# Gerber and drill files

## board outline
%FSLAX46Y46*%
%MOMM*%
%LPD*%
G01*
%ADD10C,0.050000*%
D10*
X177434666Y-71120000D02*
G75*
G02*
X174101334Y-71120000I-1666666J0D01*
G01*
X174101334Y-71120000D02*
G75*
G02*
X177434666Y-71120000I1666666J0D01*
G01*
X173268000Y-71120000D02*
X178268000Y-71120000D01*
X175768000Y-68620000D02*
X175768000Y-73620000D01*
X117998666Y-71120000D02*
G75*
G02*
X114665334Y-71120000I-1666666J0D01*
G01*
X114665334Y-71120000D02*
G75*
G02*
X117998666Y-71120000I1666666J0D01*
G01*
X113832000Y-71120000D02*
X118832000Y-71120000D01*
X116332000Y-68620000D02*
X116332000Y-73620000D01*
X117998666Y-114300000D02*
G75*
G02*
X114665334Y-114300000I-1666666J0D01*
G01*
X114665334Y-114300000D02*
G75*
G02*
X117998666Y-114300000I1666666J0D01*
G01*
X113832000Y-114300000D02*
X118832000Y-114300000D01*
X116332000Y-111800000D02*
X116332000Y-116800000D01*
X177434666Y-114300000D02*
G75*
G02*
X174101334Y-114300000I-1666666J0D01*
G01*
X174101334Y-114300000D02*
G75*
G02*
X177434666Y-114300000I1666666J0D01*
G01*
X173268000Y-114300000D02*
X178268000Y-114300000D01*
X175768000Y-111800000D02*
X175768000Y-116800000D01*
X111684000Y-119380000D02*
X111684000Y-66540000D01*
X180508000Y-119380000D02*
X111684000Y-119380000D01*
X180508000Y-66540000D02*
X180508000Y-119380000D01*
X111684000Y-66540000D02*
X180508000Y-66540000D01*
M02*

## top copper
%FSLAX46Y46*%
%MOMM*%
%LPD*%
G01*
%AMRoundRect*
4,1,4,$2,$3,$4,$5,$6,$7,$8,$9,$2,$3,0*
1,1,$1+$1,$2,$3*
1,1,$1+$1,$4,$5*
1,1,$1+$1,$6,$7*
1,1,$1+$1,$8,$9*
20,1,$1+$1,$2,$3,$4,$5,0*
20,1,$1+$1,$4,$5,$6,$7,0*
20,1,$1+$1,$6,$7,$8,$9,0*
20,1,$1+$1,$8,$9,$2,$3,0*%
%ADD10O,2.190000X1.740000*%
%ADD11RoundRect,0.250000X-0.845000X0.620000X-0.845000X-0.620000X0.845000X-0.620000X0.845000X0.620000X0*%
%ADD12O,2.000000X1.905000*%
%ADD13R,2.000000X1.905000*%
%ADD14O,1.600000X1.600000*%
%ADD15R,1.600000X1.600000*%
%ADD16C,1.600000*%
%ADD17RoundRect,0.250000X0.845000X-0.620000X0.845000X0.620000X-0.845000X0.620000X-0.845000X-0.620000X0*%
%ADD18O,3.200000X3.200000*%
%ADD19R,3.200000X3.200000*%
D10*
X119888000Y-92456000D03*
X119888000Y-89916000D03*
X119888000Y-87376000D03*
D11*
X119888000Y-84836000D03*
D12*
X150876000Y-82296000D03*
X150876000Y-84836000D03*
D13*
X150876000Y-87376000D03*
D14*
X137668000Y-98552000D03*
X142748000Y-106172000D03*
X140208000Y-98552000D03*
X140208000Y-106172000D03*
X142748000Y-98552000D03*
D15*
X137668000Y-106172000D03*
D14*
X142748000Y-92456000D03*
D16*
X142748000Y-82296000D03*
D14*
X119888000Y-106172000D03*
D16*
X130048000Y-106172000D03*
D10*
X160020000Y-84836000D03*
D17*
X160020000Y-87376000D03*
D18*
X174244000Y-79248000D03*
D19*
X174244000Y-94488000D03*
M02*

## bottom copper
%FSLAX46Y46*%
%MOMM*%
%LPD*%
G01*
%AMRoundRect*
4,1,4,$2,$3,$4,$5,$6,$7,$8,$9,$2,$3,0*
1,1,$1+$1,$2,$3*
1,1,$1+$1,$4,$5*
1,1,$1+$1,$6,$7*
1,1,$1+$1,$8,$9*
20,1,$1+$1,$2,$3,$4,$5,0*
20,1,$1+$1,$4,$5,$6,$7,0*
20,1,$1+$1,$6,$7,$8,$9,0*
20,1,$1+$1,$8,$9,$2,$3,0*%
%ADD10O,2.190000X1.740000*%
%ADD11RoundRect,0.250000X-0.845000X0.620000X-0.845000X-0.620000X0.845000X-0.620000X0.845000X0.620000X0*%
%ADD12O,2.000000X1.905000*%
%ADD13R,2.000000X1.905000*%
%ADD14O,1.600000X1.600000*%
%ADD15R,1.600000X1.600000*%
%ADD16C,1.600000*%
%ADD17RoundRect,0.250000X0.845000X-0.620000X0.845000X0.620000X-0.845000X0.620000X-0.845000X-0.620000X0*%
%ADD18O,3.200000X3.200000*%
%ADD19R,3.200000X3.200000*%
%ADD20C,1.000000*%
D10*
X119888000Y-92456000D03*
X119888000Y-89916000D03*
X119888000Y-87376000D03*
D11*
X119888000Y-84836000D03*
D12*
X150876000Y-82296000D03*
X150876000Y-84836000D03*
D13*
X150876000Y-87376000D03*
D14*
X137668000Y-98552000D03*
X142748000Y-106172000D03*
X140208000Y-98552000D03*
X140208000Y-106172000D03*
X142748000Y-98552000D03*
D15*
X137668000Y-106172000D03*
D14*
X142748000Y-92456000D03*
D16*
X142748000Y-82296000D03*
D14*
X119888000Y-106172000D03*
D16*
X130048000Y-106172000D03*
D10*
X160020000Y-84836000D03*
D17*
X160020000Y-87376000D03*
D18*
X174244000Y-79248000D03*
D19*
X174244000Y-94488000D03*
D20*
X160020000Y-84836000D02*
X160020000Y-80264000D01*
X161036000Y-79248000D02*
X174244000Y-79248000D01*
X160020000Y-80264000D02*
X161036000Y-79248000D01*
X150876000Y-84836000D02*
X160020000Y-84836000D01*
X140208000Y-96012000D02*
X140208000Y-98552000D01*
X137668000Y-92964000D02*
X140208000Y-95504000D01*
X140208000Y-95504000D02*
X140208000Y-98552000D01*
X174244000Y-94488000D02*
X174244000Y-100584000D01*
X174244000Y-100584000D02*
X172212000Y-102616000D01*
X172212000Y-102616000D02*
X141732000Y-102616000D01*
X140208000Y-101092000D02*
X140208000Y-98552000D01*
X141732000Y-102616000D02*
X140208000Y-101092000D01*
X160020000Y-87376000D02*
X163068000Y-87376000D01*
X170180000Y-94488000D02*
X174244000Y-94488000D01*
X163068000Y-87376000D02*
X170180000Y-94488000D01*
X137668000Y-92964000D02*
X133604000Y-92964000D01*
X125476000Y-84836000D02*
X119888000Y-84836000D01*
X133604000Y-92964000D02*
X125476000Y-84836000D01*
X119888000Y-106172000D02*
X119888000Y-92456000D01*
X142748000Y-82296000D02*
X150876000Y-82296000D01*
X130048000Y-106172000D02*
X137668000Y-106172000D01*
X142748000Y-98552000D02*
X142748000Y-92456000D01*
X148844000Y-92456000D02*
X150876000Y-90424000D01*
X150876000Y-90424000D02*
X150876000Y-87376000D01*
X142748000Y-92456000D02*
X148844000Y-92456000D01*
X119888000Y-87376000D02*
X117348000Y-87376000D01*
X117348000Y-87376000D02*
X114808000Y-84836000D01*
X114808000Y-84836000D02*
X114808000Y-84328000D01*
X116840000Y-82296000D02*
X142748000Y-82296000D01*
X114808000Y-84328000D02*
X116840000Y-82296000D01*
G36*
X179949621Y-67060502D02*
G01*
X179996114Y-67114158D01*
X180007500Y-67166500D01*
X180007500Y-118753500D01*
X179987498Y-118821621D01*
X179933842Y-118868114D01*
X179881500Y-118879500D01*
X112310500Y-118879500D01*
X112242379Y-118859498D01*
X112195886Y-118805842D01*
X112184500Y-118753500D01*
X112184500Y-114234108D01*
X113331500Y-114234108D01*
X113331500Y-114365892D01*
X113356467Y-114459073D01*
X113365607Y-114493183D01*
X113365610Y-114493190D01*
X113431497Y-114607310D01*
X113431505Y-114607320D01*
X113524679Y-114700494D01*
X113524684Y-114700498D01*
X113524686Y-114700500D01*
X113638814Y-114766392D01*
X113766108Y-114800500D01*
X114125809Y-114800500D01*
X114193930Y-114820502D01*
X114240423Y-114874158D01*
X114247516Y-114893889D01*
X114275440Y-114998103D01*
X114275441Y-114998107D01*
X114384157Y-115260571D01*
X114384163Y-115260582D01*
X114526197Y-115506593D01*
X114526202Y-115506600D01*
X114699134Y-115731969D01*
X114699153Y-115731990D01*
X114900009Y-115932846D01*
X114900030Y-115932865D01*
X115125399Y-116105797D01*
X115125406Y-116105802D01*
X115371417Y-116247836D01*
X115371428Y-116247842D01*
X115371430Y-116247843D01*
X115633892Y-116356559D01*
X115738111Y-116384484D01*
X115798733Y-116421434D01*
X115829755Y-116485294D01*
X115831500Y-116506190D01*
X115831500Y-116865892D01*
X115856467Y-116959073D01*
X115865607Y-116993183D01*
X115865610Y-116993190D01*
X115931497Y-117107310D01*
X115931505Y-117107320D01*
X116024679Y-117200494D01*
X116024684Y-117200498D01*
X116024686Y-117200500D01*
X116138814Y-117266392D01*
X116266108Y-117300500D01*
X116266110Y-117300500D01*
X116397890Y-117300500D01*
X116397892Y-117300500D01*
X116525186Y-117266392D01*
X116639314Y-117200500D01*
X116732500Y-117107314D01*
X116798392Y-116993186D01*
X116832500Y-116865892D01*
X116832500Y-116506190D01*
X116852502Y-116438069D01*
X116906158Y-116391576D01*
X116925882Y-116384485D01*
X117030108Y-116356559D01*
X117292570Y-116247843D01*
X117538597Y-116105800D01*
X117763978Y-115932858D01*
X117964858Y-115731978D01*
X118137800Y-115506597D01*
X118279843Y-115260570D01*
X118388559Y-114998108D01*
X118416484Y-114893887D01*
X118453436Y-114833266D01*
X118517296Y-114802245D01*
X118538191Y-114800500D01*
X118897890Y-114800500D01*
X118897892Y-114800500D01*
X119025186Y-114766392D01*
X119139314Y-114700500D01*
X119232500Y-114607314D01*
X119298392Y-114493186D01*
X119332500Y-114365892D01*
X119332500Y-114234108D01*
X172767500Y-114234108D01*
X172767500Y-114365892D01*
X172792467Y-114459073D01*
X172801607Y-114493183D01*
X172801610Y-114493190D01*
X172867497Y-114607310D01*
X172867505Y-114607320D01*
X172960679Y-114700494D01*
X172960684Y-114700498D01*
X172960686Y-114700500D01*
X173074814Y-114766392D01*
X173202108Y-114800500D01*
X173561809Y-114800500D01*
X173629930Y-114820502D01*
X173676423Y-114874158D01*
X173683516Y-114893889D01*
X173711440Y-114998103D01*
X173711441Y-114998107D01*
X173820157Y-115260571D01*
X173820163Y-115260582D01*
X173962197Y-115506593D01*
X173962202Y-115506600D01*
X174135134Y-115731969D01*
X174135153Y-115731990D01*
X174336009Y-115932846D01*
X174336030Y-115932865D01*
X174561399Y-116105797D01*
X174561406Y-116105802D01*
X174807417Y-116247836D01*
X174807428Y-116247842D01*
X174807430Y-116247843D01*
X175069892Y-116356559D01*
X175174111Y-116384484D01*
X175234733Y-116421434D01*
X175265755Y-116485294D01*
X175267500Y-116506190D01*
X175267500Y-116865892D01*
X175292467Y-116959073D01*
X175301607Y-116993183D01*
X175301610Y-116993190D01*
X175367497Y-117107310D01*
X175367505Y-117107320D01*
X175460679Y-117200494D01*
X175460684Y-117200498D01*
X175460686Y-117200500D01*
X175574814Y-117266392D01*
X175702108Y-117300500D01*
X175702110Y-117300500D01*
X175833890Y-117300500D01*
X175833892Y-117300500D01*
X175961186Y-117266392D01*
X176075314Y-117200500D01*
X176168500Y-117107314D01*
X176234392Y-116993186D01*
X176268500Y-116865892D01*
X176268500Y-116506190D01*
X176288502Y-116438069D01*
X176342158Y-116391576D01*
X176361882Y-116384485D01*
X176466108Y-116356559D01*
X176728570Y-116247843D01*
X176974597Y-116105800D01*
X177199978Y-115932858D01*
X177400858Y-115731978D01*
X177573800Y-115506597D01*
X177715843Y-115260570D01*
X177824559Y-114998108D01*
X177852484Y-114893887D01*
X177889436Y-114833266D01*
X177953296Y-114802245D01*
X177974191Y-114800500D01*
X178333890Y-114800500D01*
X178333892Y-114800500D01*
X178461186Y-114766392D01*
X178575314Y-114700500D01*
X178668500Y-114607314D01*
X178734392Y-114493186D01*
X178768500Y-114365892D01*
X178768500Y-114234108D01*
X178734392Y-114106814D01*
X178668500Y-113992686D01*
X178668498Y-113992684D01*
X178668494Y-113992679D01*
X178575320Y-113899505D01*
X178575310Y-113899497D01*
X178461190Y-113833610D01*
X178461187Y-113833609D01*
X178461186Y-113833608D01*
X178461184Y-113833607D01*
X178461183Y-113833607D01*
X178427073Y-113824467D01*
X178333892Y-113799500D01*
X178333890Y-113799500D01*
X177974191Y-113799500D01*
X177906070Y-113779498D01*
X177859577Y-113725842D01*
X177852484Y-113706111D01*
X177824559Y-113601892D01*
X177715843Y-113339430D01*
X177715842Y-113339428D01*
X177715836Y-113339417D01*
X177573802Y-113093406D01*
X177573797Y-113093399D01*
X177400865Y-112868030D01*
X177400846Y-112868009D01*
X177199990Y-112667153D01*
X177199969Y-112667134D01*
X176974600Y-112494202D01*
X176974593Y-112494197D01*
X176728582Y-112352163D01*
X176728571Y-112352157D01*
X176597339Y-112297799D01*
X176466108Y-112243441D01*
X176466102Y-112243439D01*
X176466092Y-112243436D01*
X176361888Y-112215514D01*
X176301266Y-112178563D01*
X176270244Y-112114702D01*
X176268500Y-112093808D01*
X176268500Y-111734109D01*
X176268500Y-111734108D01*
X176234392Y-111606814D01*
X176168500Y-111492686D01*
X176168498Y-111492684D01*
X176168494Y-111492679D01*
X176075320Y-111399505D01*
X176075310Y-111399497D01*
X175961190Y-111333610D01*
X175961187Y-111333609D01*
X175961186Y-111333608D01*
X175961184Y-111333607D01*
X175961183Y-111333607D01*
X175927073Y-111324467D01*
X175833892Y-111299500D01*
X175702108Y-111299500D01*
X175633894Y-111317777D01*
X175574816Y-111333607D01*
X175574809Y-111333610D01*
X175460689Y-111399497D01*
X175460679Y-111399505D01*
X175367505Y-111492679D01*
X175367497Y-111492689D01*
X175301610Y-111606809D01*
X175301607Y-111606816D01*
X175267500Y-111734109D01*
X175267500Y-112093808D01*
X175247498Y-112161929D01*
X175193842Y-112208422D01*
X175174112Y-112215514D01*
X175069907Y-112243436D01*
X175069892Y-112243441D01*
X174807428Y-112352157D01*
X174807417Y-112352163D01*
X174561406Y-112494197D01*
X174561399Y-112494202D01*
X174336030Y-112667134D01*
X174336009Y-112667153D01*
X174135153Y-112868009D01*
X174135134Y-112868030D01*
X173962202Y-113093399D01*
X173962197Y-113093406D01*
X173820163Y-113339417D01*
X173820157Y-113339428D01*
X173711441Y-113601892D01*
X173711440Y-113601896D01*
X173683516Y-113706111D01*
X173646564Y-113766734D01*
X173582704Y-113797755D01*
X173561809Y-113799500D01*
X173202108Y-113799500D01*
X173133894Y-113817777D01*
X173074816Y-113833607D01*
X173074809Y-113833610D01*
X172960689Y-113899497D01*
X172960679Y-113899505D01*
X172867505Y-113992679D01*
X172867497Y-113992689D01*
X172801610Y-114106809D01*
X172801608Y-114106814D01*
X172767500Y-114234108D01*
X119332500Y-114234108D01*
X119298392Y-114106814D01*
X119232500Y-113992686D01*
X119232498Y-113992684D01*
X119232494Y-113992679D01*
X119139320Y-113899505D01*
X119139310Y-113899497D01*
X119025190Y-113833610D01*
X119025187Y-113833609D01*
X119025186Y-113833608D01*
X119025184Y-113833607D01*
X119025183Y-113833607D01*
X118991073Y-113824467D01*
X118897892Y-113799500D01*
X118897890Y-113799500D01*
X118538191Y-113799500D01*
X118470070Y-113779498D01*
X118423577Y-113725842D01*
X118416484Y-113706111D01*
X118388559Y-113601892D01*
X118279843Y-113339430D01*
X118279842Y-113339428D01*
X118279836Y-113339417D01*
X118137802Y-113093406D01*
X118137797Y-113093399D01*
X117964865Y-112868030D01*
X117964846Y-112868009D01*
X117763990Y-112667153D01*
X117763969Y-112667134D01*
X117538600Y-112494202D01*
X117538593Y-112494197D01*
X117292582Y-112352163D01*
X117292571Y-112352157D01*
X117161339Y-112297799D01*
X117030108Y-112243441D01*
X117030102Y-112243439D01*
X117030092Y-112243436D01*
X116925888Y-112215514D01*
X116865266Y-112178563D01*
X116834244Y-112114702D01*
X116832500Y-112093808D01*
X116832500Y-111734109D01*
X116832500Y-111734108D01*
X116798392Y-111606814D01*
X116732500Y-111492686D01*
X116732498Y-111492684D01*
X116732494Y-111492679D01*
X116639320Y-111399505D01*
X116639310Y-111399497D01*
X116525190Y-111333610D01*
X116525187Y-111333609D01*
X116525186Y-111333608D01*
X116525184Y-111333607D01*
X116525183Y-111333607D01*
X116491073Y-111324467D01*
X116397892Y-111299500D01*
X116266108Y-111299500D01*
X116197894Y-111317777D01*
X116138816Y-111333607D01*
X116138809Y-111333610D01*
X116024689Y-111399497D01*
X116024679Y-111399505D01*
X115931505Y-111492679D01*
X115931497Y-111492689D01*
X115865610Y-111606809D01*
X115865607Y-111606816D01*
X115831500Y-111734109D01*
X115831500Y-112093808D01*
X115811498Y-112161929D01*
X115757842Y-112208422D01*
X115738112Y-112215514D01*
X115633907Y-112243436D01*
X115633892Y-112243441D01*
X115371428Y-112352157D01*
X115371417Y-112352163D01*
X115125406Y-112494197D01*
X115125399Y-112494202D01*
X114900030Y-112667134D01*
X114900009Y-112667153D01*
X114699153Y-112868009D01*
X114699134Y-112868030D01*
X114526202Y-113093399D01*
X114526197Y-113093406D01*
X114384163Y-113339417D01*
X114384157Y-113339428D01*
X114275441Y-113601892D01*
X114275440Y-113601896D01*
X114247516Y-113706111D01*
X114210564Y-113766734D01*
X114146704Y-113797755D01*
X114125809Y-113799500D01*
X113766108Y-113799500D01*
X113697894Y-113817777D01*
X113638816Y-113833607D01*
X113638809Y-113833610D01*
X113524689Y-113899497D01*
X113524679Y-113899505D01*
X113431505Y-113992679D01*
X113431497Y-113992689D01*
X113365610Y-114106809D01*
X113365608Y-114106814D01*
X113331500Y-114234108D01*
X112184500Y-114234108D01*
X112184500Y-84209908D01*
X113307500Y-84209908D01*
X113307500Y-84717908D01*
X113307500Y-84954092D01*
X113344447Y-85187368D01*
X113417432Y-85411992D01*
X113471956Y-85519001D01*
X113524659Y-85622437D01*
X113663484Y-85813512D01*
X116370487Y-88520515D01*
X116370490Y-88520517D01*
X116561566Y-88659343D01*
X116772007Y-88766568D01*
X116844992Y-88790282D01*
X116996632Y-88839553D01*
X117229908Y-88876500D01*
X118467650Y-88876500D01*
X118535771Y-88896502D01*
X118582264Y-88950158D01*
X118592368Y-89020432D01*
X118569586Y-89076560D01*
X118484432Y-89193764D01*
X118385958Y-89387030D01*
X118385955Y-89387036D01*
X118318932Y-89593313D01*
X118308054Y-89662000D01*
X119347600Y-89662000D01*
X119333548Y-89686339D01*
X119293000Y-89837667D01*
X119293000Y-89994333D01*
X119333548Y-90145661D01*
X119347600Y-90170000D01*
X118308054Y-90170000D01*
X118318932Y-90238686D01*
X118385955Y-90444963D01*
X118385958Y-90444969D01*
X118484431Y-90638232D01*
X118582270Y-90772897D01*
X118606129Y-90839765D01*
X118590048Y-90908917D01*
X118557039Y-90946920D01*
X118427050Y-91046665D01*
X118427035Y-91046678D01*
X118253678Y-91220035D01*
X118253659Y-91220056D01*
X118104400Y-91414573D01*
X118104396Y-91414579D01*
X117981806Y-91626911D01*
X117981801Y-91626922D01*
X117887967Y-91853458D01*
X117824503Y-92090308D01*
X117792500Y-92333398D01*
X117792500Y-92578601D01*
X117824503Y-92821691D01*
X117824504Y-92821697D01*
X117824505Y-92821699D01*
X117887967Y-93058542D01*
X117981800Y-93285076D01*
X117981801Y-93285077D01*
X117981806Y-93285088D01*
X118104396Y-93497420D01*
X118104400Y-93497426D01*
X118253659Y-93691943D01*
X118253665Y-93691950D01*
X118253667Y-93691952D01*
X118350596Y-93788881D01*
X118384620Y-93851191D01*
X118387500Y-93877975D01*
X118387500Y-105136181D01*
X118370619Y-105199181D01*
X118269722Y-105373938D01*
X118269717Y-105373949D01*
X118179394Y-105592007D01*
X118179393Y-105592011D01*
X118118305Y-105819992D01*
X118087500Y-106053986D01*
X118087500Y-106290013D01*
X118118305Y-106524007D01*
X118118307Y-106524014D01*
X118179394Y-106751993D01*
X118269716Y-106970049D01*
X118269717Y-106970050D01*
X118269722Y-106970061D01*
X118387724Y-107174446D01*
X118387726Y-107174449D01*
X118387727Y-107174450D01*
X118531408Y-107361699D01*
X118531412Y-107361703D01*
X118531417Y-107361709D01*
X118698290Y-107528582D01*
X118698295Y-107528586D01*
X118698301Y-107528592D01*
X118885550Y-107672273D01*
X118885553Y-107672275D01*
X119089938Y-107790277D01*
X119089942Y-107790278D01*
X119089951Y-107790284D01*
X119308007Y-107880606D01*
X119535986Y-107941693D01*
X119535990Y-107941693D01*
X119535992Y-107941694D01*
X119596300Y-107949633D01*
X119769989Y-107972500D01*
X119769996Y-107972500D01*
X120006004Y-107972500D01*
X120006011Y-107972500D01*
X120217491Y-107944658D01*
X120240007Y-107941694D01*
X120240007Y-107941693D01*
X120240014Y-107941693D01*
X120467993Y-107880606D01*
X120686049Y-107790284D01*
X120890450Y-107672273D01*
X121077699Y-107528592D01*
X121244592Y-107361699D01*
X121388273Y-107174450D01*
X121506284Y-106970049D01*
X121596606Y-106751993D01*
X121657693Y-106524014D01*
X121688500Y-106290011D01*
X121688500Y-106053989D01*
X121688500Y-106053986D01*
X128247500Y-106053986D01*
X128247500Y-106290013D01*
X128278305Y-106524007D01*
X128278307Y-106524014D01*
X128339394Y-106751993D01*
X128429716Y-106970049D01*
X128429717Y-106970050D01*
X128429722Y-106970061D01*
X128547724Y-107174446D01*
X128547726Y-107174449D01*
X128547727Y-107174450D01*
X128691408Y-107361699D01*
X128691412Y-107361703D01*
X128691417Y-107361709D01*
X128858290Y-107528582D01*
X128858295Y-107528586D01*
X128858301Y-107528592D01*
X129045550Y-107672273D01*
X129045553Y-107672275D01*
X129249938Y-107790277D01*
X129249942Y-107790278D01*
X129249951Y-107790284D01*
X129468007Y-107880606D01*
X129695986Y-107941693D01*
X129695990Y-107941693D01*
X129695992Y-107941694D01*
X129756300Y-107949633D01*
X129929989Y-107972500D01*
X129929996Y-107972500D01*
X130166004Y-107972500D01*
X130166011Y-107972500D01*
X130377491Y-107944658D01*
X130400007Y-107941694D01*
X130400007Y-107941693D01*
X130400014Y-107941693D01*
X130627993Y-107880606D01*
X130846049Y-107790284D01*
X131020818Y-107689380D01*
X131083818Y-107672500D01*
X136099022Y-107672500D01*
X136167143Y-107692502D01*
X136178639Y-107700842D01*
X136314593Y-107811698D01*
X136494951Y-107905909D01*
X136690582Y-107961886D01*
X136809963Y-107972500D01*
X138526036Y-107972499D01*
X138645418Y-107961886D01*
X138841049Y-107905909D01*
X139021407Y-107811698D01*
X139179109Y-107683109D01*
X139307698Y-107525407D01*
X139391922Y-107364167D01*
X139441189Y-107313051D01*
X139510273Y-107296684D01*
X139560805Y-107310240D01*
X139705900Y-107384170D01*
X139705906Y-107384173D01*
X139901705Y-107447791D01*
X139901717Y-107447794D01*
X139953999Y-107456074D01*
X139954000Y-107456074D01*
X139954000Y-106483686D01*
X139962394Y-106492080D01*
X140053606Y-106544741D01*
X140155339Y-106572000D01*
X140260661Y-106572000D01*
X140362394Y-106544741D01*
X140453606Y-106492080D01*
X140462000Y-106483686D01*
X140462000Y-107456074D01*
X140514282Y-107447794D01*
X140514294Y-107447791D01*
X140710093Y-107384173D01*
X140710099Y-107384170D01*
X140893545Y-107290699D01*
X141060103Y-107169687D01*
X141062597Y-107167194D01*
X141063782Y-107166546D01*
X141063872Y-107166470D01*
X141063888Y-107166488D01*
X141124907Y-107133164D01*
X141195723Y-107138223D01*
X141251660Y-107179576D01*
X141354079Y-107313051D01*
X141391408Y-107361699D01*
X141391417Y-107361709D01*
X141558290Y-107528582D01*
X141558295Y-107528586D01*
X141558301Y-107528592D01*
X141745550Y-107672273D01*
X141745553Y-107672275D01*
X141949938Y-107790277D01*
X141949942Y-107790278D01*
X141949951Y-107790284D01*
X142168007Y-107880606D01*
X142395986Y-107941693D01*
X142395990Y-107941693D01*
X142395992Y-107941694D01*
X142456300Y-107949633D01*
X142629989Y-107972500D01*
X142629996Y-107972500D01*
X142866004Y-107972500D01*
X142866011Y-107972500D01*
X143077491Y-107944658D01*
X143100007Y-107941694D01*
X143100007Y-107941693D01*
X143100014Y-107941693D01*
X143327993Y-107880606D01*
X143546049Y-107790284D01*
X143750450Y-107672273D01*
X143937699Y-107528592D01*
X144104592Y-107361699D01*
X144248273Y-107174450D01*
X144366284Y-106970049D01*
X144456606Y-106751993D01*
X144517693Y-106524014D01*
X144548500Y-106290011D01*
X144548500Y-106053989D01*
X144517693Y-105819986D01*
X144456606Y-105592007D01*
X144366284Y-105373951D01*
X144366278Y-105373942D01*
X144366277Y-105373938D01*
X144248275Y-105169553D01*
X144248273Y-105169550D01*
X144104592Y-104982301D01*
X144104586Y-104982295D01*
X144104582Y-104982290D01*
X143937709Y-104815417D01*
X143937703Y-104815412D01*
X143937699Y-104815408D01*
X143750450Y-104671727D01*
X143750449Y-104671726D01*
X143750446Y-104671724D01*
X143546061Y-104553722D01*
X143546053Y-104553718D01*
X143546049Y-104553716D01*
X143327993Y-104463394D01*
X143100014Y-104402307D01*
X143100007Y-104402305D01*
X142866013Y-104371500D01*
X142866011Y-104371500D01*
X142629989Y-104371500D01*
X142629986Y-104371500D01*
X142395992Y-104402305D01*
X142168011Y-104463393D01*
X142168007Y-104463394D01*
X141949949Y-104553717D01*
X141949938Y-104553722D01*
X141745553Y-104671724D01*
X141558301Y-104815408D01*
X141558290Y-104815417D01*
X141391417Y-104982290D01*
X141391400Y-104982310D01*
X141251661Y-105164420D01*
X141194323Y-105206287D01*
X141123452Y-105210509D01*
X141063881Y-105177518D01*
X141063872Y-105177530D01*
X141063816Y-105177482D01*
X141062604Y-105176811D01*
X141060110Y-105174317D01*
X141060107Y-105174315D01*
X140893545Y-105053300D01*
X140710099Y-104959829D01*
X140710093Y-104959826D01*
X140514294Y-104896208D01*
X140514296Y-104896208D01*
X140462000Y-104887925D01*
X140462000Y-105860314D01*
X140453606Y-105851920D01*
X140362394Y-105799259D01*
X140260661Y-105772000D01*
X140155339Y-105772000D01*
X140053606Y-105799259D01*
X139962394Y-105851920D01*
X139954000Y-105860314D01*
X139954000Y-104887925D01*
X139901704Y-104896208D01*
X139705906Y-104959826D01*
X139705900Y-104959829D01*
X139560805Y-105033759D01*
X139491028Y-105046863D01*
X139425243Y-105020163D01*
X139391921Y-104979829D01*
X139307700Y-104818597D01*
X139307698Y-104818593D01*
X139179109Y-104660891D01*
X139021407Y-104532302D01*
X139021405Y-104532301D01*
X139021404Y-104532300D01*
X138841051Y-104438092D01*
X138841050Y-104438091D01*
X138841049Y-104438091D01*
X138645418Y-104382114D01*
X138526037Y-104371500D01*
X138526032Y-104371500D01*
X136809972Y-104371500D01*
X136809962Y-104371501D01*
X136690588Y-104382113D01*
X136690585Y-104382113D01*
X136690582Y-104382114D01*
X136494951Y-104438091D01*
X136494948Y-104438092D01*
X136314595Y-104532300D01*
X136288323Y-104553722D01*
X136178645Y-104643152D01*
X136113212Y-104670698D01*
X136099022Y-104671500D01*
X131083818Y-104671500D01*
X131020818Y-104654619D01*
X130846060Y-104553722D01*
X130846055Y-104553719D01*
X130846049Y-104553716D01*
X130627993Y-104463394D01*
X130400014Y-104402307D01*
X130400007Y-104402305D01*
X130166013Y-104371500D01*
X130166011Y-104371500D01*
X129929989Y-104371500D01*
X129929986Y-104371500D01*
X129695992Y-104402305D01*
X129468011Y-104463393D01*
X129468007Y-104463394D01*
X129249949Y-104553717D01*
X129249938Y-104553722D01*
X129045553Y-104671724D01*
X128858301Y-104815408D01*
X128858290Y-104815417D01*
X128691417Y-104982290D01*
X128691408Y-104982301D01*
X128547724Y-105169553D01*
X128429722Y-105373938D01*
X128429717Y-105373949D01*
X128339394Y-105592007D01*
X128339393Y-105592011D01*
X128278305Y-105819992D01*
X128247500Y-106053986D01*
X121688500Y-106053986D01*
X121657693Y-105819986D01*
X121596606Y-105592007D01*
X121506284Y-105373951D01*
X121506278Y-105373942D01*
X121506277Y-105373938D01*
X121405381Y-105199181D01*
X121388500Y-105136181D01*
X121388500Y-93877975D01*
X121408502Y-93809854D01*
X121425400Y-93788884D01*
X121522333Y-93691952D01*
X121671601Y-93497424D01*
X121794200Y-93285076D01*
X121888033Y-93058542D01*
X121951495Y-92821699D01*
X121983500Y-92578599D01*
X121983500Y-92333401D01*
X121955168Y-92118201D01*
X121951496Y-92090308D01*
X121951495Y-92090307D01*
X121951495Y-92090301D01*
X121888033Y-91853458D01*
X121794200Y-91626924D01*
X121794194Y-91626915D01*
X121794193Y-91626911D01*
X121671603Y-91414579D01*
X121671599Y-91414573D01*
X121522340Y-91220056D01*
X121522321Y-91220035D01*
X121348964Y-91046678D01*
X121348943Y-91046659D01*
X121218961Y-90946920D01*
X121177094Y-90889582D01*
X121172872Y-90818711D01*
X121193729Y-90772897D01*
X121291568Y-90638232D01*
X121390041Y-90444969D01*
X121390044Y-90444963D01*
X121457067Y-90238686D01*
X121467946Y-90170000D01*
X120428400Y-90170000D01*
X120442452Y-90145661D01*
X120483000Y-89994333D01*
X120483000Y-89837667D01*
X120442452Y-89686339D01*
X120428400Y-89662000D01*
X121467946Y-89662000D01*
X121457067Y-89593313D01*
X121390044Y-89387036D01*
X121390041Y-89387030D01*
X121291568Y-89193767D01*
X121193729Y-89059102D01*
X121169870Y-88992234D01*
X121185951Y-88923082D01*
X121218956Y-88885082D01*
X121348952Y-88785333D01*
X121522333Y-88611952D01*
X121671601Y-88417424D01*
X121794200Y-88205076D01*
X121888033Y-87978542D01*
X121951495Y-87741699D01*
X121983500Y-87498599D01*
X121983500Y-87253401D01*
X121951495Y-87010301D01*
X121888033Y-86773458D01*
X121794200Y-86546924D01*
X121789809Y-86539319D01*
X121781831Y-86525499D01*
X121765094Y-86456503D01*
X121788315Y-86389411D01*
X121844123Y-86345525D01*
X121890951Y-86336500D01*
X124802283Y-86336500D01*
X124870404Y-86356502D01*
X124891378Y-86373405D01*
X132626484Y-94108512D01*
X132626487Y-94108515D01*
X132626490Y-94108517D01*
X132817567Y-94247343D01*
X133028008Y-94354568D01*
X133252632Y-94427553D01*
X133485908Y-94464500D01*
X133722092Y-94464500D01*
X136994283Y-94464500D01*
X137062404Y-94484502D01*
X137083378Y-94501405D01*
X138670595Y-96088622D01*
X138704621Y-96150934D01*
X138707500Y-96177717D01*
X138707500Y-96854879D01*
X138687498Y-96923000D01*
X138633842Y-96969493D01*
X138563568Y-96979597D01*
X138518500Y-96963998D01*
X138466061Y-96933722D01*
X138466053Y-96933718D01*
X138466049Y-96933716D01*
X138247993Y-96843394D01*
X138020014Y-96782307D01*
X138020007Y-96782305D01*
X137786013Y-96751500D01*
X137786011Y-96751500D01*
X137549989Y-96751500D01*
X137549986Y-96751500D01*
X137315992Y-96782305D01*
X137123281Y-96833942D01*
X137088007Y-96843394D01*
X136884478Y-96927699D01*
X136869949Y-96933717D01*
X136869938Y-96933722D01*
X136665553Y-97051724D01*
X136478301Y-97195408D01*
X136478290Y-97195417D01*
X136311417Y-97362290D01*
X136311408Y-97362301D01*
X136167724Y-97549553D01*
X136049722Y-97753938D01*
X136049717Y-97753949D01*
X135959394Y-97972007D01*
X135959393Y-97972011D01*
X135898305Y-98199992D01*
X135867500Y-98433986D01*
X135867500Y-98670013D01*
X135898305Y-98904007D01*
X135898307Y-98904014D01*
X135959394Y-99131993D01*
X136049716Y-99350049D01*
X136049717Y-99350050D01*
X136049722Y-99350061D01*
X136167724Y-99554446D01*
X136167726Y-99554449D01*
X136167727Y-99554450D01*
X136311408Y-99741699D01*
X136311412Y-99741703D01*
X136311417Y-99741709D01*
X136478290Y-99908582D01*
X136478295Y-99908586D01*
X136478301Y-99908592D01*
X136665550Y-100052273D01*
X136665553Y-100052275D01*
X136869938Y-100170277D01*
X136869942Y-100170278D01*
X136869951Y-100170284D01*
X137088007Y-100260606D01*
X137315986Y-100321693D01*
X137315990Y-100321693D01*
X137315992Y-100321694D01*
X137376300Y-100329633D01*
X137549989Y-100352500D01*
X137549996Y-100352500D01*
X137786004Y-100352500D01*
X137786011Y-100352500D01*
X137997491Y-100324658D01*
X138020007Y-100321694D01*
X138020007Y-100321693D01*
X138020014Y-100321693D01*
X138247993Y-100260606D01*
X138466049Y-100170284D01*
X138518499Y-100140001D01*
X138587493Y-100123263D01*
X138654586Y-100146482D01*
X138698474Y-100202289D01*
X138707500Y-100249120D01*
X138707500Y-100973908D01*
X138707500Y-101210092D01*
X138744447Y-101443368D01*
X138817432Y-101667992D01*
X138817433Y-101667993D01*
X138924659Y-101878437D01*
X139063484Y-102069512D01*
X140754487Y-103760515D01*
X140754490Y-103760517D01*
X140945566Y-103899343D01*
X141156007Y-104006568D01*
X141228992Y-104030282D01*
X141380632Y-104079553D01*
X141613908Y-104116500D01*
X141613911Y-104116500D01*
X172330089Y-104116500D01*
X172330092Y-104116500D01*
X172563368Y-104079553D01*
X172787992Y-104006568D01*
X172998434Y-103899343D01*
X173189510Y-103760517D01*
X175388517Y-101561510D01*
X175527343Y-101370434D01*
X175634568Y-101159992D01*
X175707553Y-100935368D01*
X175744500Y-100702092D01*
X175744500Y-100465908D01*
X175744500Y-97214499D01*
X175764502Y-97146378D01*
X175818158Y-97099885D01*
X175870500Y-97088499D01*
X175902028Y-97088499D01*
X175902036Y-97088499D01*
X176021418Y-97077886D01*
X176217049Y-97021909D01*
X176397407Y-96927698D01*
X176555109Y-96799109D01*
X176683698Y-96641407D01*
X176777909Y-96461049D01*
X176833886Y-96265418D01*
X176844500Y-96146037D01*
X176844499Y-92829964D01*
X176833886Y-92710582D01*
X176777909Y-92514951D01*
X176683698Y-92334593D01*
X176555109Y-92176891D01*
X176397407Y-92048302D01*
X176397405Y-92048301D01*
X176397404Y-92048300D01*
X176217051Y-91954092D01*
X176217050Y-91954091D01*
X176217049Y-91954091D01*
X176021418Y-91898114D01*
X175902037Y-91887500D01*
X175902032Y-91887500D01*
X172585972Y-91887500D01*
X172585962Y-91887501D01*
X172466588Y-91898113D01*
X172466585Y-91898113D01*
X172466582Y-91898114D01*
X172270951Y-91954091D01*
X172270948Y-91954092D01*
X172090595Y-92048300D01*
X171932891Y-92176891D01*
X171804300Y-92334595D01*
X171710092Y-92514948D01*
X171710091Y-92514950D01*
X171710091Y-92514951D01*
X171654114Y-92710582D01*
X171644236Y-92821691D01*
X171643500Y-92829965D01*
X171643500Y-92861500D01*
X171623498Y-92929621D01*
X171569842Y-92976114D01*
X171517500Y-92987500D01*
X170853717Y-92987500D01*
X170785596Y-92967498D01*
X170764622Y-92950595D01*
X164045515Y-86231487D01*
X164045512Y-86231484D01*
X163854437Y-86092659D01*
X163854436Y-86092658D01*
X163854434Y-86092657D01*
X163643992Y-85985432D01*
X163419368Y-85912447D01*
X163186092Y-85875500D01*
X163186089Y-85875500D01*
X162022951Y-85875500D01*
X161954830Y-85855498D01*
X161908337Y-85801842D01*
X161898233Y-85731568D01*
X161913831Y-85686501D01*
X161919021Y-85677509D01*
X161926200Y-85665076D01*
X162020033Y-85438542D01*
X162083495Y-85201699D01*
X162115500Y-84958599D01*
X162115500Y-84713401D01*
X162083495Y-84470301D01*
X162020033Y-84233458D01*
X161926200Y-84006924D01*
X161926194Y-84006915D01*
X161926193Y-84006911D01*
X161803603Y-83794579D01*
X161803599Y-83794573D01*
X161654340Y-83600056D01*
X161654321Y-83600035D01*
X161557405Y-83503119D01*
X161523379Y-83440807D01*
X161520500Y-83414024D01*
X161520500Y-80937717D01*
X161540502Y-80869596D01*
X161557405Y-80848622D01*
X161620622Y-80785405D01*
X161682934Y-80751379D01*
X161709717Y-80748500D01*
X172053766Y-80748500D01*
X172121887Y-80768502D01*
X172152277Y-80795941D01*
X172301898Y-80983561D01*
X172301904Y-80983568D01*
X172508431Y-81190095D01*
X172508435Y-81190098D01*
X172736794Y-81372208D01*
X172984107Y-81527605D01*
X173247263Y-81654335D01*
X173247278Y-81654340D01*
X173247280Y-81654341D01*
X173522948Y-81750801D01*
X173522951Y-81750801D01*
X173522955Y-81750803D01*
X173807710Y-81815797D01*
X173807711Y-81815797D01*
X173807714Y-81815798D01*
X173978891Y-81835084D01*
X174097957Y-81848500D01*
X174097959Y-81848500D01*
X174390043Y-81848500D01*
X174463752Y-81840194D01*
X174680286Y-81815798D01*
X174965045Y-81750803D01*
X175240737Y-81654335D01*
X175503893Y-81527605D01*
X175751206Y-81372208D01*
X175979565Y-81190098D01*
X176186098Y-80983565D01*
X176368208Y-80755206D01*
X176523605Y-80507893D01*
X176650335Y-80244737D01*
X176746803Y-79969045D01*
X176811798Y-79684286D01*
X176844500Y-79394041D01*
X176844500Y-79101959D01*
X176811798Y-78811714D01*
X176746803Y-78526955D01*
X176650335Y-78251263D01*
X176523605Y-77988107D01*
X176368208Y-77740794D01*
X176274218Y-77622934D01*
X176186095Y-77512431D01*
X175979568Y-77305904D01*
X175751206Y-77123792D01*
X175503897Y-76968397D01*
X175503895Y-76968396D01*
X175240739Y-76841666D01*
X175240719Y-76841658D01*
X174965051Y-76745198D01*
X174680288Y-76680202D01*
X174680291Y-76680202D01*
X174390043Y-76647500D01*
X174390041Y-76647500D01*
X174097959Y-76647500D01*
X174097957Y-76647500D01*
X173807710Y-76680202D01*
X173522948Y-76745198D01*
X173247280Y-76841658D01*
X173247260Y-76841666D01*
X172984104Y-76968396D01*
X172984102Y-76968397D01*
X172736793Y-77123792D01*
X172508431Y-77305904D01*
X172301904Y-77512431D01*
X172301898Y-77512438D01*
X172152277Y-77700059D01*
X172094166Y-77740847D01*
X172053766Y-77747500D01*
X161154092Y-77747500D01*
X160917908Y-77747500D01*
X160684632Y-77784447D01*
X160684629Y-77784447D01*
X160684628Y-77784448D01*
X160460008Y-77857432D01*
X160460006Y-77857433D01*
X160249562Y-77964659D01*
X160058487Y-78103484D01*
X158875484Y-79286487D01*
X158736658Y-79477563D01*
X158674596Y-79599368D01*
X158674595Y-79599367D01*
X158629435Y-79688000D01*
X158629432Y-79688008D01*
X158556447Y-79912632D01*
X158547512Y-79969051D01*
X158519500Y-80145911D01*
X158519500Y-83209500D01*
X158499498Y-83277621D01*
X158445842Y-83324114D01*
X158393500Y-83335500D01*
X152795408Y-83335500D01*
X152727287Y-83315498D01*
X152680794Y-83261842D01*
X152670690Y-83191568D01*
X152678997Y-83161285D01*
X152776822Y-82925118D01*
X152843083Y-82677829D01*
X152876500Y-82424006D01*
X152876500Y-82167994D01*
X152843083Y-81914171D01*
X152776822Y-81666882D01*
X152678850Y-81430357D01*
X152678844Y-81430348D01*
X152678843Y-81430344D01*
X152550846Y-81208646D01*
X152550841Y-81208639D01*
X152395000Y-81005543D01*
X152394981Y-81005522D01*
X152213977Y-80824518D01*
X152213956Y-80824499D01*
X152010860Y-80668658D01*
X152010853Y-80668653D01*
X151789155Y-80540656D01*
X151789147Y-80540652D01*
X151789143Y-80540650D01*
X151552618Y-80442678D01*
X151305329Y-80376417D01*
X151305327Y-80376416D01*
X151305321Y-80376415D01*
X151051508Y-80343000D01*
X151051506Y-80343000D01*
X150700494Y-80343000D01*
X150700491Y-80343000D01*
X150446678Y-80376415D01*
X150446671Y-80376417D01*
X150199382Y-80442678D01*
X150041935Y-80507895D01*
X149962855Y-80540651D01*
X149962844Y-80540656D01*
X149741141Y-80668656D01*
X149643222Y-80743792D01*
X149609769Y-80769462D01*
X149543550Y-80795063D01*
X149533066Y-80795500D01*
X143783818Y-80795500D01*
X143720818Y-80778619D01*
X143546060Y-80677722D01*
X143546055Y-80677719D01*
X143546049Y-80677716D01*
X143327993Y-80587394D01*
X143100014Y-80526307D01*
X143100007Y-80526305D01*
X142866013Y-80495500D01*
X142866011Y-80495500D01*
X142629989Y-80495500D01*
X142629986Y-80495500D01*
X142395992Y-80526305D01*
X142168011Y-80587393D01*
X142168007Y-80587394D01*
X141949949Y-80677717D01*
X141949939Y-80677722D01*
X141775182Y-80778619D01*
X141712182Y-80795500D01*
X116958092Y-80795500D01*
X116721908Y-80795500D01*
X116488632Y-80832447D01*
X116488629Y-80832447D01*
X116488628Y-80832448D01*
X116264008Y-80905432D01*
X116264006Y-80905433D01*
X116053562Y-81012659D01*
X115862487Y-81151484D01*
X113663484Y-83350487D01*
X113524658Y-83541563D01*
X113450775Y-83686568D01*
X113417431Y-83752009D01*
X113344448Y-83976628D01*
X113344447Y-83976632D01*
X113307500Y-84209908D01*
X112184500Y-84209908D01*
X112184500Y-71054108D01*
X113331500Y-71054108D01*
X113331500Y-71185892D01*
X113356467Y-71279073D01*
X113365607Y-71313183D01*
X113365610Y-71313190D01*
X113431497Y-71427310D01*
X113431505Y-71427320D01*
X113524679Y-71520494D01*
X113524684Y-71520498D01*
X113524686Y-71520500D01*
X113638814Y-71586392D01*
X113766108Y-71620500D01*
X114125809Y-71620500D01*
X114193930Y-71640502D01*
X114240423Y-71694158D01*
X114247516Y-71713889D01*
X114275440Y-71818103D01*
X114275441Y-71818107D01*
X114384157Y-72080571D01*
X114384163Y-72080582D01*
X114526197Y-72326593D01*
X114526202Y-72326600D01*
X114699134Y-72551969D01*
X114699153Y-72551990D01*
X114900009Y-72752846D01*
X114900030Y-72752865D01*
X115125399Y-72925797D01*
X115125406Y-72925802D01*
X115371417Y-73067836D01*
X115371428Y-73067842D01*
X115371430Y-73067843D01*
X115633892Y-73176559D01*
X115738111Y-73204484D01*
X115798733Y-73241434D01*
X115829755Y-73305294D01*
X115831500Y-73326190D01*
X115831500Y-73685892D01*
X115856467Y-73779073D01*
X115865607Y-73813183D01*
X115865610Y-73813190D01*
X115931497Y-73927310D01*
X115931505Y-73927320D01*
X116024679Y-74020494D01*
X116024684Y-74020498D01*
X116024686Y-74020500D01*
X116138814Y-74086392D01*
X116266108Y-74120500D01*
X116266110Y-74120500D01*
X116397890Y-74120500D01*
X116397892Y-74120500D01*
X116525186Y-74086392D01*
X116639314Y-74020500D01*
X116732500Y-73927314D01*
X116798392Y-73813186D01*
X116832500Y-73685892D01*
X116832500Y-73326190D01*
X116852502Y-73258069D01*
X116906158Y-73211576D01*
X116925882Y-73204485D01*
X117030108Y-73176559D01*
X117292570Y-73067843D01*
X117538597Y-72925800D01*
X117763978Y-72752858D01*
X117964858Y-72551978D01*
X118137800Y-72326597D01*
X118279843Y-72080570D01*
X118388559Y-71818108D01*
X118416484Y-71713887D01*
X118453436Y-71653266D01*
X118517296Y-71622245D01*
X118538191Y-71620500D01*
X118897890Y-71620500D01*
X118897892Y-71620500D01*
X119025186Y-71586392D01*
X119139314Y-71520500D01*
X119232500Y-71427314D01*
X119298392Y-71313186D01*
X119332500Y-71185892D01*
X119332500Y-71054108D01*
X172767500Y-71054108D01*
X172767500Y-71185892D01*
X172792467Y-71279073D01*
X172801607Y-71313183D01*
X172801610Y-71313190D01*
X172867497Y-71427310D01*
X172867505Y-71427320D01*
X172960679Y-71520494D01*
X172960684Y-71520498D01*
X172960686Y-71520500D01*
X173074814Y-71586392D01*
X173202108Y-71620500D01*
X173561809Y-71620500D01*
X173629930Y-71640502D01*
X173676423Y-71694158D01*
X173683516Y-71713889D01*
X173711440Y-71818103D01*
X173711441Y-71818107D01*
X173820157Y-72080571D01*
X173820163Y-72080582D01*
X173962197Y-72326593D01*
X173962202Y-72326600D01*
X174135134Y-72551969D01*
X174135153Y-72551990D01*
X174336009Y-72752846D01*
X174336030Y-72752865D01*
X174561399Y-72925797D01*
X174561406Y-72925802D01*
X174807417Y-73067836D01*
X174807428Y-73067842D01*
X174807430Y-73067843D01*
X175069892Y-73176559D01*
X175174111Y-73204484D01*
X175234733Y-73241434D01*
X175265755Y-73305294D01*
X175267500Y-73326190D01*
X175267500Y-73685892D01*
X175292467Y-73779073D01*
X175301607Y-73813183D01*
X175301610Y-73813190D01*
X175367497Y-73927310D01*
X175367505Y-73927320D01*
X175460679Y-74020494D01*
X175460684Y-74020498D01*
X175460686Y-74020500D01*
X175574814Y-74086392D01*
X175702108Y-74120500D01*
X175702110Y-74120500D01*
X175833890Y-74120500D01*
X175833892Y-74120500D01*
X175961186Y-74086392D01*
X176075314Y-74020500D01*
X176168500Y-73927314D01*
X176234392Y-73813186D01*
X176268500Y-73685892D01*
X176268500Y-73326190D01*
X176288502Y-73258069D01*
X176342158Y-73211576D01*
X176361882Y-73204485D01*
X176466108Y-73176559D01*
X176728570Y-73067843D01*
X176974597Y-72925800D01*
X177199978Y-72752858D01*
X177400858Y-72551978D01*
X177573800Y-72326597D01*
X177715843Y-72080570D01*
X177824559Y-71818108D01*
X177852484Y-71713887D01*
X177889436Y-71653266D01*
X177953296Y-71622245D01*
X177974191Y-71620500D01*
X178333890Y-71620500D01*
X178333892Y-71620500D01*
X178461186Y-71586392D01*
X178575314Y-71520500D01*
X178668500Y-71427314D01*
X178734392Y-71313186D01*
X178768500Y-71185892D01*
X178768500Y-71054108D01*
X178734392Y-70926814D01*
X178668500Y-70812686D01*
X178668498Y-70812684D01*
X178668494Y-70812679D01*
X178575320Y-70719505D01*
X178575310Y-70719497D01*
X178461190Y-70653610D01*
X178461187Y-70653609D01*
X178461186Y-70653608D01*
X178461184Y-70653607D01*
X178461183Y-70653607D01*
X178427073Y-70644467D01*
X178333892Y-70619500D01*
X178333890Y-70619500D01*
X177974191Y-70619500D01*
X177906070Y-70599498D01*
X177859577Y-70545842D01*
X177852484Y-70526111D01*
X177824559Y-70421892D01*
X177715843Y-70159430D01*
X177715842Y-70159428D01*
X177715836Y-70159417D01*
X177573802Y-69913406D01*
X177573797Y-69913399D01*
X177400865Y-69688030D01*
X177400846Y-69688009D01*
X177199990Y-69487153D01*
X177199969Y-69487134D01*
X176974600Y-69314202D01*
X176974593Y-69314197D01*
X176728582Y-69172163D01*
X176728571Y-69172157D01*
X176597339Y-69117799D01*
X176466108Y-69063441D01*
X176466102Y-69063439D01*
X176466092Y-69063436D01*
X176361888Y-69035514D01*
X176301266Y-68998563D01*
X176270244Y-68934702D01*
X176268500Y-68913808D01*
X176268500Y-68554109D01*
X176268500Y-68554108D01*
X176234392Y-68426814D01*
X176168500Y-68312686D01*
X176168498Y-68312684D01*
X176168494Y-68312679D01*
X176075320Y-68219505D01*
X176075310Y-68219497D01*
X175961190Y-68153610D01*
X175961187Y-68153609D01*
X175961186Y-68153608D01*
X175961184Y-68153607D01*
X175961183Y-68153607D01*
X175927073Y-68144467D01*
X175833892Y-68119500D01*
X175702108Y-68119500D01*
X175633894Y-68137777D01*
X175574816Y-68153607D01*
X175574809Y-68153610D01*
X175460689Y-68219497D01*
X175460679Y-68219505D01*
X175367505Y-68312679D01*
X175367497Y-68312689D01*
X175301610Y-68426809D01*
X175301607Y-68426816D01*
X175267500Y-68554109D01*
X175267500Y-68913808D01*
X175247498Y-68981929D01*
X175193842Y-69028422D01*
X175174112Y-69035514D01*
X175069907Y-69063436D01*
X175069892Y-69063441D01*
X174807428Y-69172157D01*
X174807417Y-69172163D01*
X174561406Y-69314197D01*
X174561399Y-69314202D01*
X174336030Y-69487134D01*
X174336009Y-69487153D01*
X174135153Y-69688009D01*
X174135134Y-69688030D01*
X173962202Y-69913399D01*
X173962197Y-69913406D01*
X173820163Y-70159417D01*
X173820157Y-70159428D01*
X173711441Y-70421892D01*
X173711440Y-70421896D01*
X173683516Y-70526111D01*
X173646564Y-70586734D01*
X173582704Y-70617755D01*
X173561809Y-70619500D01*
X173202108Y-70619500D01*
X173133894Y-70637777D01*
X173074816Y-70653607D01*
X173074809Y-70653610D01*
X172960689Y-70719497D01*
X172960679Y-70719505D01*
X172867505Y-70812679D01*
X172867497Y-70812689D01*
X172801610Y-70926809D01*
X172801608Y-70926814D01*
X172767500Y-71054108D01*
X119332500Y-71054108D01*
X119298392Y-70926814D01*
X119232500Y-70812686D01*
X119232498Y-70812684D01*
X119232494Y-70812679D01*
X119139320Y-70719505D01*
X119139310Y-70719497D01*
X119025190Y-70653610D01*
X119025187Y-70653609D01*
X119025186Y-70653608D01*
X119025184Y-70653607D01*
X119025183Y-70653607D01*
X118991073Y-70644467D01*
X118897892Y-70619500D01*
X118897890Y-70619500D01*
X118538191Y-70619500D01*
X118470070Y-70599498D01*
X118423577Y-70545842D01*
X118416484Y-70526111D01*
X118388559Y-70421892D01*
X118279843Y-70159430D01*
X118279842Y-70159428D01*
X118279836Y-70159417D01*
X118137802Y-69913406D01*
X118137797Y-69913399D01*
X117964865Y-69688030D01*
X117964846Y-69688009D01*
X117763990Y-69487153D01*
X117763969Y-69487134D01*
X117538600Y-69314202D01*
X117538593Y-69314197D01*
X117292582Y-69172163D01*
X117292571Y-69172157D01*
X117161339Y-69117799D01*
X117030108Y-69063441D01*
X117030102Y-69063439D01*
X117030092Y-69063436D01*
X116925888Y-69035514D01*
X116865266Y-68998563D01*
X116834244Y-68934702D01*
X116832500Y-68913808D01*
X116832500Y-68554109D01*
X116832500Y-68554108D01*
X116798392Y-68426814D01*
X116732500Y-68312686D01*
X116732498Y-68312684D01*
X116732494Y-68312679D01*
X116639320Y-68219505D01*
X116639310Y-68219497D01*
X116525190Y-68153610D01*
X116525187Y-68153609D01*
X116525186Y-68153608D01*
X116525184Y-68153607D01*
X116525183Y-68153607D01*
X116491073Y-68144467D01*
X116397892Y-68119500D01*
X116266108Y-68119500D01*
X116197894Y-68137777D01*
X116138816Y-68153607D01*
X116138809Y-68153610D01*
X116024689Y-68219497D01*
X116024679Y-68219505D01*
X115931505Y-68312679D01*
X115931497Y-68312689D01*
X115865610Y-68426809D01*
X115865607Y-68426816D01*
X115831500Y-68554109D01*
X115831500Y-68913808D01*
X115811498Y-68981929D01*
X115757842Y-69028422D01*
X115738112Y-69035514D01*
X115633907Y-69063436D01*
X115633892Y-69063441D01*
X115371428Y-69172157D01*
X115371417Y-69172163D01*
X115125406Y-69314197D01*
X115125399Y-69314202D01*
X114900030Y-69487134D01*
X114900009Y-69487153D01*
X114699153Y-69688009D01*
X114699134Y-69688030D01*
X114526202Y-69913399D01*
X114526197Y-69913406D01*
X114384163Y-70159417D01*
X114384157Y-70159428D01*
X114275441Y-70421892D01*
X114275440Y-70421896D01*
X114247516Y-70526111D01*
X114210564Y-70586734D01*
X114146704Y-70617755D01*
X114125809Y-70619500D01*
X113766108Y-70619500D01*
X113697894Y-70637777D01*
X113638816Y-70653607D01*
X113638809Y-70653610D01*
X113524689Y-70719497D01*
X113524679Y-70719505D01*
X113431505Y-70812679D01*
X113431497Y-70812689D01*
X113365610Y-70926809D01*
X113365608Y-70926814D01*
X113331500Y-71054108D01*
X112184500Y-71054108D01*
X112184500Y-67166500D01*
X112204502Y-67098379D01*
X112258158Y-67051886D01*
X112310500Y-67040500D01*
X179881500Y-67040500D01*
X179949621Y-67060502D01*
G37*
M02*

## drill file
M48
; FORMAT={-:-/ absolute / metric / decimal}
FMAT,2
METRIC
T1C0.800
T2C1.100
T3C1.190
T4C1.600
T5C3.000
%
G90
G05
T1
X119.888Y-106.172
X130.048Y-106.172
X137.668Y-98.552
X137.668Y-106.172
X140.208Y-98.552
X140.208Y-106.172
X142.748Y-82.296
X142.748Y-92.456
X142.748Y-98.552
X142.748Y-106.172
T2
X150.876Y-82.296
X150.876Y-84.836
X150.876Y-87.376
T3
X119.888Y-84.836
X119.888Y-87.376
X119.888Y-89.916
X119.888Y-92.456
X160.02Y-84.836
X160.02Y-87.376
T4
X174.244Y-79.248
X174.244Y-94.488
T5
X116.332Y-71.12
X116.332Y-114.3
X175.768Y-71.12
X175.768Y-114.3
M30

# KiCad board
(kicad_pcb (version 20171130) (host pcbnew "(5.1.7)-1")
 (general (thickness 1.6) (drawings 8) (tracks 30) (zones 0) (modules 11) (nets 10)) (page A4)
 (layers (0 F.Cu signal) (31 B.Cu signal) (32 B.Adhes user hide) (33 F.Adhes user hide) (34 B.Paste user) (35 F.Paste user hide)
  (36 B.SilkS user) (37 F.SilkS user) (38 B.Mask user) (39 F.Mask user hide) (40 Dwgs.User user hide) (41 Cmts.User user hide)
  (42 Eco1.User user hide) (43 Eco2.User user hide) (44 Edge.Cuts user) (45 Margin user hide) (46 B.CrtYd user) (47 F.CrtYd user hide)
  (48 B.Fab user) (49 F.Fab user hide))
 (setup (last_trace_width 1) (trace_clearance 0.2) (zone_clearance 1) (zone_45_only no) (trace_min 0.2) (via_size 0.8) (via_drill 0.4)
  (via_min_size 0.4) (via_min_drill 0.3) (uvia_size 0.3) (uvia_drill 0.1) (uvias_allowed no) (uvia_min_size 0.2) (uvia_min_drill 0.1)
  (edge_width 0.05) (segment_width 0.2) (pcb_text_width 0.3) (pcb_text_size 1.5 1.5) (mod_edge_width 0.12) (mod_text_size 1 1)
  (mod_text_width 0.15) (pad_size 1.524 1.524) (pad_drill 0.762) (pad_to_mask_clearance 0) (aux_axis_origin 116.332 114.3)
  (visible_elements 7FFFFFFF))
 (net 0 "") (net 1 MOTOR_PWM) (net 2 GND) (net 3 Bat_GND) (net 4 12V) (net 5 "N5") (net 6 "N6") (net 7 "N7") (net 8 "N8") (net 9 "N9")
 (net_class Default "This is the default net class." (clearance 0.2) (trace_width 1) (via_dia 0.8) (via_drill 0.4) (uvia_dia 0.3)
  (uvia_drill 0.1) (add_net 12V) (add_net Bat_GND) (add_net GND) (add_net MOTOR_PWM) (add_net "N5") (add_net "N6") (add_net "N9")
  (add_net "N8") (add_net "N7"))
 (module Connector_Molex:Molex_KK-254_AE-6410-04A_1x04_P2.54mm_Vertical (layer F.Cu) (at 119.888 84.836 270)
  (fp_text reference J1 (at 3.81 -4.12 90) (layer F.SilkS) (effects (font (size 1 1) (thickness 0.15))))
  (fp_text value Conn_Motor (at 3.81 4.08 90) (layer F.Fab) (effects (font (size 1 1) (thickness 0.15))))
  (pad 4 thru_hole oval (at 7.62 0 270) (size 1.74 2.19) (drill 1.19) (layers *.Cu *.Mask) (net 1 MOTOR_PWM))
  (pad 3 thru_hole oval (at 5.08 0 270) (size 1.74 2.19) (drill 1.19) (layers *.Cu *.Mask) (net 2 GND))
  (pad 2 thru_hole oval (at 2.54 0 270) (size 1.74 2.19) (drill 1.19) (layers *.Cu *.Mask) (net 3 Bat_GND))
  (pad 1 thru_hole roundrect (at 0 0 270) (size 1.74 2.19) (drill 1.19) (layers *.Cu *.Mask) (roundrect_rratio 0.143678) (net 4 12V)))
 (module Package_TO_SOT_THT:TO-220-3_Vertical (layer F.Cu) (at 150.876 87.376 90)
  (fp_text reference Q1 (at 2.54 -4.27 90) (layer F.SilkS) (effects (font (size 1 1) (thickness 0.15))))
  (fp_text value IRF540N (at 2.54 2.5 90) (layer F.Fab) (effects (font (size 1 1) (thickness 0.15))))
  (pad 3 thru_hole oval (at 5.08 0 90) (size 1.905 2) (drill 1.1) (layers *.Cu *.Mask) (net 3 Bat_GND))
  (pad 2 thru_hole oval (at 2.54 0 90) (size 1.905 2) (drill 1.1) (layers *.Cu *.Mask) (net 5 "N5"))
  (pad 1 thru_hole rect (at 0 0 90) (size 1.905 2) (drill 1.1) (layers *.Cu *.Mask) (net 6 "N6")))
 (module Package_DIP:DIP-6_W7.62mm (layer F.Cu) (at 137.668 106.172 90)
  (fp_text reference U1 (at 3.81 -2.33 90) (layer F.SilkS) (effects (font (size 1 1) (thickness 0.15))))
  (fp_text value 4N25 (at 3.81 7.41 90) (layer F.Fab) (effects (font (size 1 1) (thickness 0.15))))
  (pad 6 thru_hole oval (at 7.62 0 90) (size 1.6 1.6) (drill 0.8) (layers *.Cu *.Mask) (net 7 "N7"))
  (pad 3 thru_hole oval (at 0 5.08 90) (size 1.6 1.6) (drill 0.8) (layers *.Cu *.Mask) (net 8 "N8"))
  (pad 5 thru_hole oval (at 7.62 2.54 90) (size 1.6 1.6) (drill 0.8) (layers *.Cu *.Mask) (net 4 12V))
  (pad 2 thru_hole oval (at 0 2.54 90) (size 1.6 1.6) (drill 0.8) (layers *.Cu *.Mask) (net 2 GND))
  (pad 4 thru_hole oval (at 7.62 5.08 90) (size 1.6 1.6) (drill 0.8) (layers *.Cu *.Mask) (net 6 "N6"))
  (pad 1 thru_hole rect (at 0 0 90) (size 1.6 1.6) (drill 0.8) (layers *.Cu *.Mask) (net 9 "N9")))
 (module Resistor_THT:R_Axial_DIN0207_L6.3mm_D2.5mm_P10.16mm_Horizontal (layer F.Cu) (at 142.748 82.296 270)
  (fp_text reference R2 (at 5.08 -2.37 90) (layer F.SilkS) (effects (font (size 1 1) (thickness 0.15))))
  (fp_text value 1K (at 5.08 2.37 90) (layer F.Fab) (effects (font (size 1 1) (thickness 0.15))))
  (pad 2 thru_hole oval (at 10.16 0 270) (size 1.6 1.6) (drill 0.8) (layers *.Cu *.Mask) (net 6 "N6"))
  (pad 1 thru_hole circle (at 0 0 270) (size 1.6 1.6) (drill 0.8) (layers *.Cu *.Mask) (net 3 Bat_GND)))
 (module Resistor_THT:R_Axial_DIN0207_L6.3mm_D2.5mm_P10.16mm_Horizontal (layer F.Cu) (at 130.048 106.172 180)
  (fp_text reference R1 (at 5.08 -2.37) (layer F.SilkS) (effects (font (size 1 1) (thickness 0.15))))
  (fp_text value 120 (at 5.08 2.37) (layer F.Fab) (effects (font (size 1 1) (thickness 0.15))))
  (pad 2 thru_hole oval (at 10.16 0 180) (size 1.6 1.6) (drill 0.8) (layers *.Cu *.Mask) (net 1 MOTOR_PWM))
  (pad 1 thru_hole circle (at 0 0 180) (size 1.6 1.6) (drill 0.8) (layers *.Cu *.Mask) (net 9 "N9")))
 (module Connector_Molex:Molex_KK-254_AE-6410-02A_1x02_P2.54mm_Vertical (layer F.Cu) (at 160.02 87.376 90)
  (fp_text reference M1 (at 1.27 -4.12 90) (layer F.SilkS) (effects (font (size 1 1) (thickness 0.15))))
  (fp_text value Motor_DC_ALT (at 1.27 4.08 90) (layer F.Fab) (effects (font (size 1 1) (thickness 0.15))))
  (pad 2 thru_hole oval (at 2.54 0 90) (size 1.74 2.19) (drill 1.19) (layers *.Cu *.Mask) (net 5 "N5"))
  (pad 1 thru_hole roundrect (at 0 0 90) (size 1.74 2.19) (drill 1.19) (layers *.Cu *.Mask) (roundrect_rratio 0.143678) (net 4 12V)))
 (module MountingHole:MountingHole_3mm (layer F.Cu) (at 116.332 114.3)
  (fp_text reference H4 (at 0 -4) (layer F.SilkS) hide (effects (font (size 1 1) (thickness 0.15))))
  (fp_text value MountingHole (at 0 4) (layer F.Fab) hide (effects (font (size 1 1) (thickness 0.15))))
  (pad 1 np_thru_hole circle (at 0 0) (size 3 3) (drill 3) (layers *.Cu *.Mask)))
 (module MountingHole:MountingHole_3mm (layer F.Cu) (at 175.768 114.3)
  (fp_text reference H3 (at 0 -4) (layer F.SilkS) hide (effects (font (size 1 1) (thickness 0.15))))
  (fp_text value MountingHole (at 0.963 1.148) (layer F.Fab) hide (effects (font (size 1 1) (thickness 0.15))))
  (pad 1 np_thru_hole circle (at 0 0) (size 3 3) (drill 3) (layers *.Cu *.Mask)))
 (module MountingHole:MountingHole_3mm (layer F.Cu) (at 175.768 71.12)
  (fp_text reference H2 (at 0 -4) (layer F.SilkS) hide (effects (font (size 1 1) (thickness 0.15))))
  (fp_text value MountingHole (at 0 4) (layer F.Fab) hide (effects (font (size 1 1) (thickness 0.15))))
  (pad 1 np_thru_hole circle (at 0 0) (size 3 3) (drill 3) (layers *.Cu *.Mask)))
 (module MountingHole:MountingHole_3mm (layer F.Cu) (at 116.332 71.12)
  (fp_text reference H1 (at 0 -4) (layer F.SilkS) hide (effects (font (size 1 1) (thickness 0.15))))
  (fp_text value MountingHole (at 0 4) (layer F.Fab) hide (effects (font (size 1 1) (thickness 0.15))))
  (pad 1 np_thru_hole circle (at 0 0) (size 3 3) (drill 3) (layers *.Cu *.Mask)))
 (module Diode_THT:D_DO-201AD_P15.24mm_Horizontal (layer F.Cu) (at 174.244 94.488 90)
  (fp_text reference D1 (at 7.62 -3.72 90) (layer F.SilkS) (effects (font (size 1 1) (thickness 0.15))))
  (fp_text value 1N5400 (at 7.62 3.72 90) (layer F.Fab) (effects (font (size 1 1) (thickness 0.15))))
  (pad 2 thru_hole oval (at 15.24 0 90) (size 3.2 3.2) (drill 1.6) (layers *.Cu *.Mask) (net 5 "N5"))
  (pad 1 thru_hole rect (at 0 0 90) (size 3.2 3.2) (drill 1.6) (layers *.Cu *.Mask) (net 4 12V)))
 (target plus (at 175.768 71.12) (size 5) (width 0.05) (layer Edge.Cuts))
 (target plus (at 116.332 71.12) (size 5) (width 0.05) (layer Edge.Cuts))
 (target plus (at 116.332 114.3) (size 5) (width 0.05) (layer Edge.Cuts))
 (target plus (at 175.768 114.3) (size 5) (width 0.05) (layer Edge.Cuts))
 (gr_line (start 111.684 119.38) (end 111.684 66.54) (layer Edge.Cuts) (width 0.05))
 (gr_line (start 180.508 119.38) (end 111.684 119.38) (layer Edge.Cuts) (width 0.05))
 (gr_line (start 180.508 66.54) (end 180.508 119.38) (layer Edge.Cuts) (width 0.05))
 (gr_line (start 111.684 66.54) (end 180.508 66.54) (layer Edge.Cuts) (width 0.05))
 (segment (start 160.02 84.836) (end 160.02 80.264) (width 1) (layer B.Cu) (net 5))
 (segment (start 161.036 79.248) (end 174.244 79.248) (width 1) (layer B.Cu) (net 5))
 (segment (start 160.02 80.264) (end 161.036 79.248) (width 1) (layer B.Cu) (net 5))
 (segment (start 150.876 84.836) (end 160.02 84.836) (width 1) (layer B.Cu) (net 5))
 (segment (start 140.208 96.012) (end 140.208 98.552) (width 1) (layer B.Cu) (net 4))
 (segment (start 137.668 92.964) (end 140.208 95.504) (width 1) (layer B.Cu) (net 4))
 (segment (start 140.208 95.504) (end 140.208 98.552) (width 1) (layer B.Cu) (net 4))
 (segment (start 174.244 94.488) (end 174.244 100.584) (width 1) (layer B.Cu) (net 4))
 (segment (start 174.244 100.584) (end 172.212 102.616) (width 1) (layer B.Cu) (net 4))
 (segment (start 172.212 102.616) (end 141.732 102.616) (width 1) (layer B.Cu) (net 4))
 (segment (start 140.208 101.092) (end 140.208 98.552) (width 1) (layer B.Cu) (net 4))
 (segment (start 141.732 102.616) (end 140.208 101.092) (width 1) (layer B.Cu) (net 4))
 (segment (start 160.02 87.376) (end 163.068 87.376) (width 1) (layer B.Cu) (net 4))
 (segment (start 170.18 94.488) (end 174.244 94.488) (width 1) (layer B.Cu) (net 4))
 (segment (start 163.068 87.376) (end 170.18 94.488) (width 1) (layer B.Cu) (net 4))
 (segment (start 137.668 92.964) (end 133.604 92.964) (width 1) (layer B.Cu) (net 4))
 (segment (start 125.476 84.836) (end 119.888 84.836) (width 1) (layer B.Cu) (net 4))
 (segment (start 133.604 92.964) (end 125.476 84.836) (width 1) (layer B.Cu) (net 4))
 (segment (start 119.888 106.172) (end 119.888 92.456) (width 1) (layer B.Cu) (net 1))
 (segment (start 142.748 82.296) (end 150.876 82.296) (width 1) (layer B.Cu) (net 3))
 (segment (start 130.048 106.172) (end 137.668 106.172) (width 1) (layer B.Cu) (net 9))
 (segment (start 142.748 98.552) (end 142.748 92.456) (width 1) (layer B.Cu) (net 6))
 (segment (start 148.844 92.456) (end 150.876 90.424) (width 1) (layer B.Cu) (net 6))
 (segment (start 150.876 90.424) (end 150.876 87.376) (width 1) (layer B.Cu) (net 6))
 (segment (start 142.748 92.456) (end 148.844 92.456) (width 1) (layer B.Cu) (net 6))
 (segment (start 119.888 87.376) (end 117.348 87.376) (width 1) (layer B.Cu) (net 3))
 (segment (start 117.348 87.376) (end 114.808 84.836) (width 1) (layer B.Cu) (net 3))
 (segment (start 114.808 84.836) (end 114.808 84.328) (width 1) (layer B.Cu) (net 3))
 (segment (start 116.84 82.296) (end 142.748 82.296) (width 1) (layer B.Cu) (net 3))
 (segment (start 114.808 84.328) (end 116.84 82.296) (width 1) (layer B.Cu) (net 3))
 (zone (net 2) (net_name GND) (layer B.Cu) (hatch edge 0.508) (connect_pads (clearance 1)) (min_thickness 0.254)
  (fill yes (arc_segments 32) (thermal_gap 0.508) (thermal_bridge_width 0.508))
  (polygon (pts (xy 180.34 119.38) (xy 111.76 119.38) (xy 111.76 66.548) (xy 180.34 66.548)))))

